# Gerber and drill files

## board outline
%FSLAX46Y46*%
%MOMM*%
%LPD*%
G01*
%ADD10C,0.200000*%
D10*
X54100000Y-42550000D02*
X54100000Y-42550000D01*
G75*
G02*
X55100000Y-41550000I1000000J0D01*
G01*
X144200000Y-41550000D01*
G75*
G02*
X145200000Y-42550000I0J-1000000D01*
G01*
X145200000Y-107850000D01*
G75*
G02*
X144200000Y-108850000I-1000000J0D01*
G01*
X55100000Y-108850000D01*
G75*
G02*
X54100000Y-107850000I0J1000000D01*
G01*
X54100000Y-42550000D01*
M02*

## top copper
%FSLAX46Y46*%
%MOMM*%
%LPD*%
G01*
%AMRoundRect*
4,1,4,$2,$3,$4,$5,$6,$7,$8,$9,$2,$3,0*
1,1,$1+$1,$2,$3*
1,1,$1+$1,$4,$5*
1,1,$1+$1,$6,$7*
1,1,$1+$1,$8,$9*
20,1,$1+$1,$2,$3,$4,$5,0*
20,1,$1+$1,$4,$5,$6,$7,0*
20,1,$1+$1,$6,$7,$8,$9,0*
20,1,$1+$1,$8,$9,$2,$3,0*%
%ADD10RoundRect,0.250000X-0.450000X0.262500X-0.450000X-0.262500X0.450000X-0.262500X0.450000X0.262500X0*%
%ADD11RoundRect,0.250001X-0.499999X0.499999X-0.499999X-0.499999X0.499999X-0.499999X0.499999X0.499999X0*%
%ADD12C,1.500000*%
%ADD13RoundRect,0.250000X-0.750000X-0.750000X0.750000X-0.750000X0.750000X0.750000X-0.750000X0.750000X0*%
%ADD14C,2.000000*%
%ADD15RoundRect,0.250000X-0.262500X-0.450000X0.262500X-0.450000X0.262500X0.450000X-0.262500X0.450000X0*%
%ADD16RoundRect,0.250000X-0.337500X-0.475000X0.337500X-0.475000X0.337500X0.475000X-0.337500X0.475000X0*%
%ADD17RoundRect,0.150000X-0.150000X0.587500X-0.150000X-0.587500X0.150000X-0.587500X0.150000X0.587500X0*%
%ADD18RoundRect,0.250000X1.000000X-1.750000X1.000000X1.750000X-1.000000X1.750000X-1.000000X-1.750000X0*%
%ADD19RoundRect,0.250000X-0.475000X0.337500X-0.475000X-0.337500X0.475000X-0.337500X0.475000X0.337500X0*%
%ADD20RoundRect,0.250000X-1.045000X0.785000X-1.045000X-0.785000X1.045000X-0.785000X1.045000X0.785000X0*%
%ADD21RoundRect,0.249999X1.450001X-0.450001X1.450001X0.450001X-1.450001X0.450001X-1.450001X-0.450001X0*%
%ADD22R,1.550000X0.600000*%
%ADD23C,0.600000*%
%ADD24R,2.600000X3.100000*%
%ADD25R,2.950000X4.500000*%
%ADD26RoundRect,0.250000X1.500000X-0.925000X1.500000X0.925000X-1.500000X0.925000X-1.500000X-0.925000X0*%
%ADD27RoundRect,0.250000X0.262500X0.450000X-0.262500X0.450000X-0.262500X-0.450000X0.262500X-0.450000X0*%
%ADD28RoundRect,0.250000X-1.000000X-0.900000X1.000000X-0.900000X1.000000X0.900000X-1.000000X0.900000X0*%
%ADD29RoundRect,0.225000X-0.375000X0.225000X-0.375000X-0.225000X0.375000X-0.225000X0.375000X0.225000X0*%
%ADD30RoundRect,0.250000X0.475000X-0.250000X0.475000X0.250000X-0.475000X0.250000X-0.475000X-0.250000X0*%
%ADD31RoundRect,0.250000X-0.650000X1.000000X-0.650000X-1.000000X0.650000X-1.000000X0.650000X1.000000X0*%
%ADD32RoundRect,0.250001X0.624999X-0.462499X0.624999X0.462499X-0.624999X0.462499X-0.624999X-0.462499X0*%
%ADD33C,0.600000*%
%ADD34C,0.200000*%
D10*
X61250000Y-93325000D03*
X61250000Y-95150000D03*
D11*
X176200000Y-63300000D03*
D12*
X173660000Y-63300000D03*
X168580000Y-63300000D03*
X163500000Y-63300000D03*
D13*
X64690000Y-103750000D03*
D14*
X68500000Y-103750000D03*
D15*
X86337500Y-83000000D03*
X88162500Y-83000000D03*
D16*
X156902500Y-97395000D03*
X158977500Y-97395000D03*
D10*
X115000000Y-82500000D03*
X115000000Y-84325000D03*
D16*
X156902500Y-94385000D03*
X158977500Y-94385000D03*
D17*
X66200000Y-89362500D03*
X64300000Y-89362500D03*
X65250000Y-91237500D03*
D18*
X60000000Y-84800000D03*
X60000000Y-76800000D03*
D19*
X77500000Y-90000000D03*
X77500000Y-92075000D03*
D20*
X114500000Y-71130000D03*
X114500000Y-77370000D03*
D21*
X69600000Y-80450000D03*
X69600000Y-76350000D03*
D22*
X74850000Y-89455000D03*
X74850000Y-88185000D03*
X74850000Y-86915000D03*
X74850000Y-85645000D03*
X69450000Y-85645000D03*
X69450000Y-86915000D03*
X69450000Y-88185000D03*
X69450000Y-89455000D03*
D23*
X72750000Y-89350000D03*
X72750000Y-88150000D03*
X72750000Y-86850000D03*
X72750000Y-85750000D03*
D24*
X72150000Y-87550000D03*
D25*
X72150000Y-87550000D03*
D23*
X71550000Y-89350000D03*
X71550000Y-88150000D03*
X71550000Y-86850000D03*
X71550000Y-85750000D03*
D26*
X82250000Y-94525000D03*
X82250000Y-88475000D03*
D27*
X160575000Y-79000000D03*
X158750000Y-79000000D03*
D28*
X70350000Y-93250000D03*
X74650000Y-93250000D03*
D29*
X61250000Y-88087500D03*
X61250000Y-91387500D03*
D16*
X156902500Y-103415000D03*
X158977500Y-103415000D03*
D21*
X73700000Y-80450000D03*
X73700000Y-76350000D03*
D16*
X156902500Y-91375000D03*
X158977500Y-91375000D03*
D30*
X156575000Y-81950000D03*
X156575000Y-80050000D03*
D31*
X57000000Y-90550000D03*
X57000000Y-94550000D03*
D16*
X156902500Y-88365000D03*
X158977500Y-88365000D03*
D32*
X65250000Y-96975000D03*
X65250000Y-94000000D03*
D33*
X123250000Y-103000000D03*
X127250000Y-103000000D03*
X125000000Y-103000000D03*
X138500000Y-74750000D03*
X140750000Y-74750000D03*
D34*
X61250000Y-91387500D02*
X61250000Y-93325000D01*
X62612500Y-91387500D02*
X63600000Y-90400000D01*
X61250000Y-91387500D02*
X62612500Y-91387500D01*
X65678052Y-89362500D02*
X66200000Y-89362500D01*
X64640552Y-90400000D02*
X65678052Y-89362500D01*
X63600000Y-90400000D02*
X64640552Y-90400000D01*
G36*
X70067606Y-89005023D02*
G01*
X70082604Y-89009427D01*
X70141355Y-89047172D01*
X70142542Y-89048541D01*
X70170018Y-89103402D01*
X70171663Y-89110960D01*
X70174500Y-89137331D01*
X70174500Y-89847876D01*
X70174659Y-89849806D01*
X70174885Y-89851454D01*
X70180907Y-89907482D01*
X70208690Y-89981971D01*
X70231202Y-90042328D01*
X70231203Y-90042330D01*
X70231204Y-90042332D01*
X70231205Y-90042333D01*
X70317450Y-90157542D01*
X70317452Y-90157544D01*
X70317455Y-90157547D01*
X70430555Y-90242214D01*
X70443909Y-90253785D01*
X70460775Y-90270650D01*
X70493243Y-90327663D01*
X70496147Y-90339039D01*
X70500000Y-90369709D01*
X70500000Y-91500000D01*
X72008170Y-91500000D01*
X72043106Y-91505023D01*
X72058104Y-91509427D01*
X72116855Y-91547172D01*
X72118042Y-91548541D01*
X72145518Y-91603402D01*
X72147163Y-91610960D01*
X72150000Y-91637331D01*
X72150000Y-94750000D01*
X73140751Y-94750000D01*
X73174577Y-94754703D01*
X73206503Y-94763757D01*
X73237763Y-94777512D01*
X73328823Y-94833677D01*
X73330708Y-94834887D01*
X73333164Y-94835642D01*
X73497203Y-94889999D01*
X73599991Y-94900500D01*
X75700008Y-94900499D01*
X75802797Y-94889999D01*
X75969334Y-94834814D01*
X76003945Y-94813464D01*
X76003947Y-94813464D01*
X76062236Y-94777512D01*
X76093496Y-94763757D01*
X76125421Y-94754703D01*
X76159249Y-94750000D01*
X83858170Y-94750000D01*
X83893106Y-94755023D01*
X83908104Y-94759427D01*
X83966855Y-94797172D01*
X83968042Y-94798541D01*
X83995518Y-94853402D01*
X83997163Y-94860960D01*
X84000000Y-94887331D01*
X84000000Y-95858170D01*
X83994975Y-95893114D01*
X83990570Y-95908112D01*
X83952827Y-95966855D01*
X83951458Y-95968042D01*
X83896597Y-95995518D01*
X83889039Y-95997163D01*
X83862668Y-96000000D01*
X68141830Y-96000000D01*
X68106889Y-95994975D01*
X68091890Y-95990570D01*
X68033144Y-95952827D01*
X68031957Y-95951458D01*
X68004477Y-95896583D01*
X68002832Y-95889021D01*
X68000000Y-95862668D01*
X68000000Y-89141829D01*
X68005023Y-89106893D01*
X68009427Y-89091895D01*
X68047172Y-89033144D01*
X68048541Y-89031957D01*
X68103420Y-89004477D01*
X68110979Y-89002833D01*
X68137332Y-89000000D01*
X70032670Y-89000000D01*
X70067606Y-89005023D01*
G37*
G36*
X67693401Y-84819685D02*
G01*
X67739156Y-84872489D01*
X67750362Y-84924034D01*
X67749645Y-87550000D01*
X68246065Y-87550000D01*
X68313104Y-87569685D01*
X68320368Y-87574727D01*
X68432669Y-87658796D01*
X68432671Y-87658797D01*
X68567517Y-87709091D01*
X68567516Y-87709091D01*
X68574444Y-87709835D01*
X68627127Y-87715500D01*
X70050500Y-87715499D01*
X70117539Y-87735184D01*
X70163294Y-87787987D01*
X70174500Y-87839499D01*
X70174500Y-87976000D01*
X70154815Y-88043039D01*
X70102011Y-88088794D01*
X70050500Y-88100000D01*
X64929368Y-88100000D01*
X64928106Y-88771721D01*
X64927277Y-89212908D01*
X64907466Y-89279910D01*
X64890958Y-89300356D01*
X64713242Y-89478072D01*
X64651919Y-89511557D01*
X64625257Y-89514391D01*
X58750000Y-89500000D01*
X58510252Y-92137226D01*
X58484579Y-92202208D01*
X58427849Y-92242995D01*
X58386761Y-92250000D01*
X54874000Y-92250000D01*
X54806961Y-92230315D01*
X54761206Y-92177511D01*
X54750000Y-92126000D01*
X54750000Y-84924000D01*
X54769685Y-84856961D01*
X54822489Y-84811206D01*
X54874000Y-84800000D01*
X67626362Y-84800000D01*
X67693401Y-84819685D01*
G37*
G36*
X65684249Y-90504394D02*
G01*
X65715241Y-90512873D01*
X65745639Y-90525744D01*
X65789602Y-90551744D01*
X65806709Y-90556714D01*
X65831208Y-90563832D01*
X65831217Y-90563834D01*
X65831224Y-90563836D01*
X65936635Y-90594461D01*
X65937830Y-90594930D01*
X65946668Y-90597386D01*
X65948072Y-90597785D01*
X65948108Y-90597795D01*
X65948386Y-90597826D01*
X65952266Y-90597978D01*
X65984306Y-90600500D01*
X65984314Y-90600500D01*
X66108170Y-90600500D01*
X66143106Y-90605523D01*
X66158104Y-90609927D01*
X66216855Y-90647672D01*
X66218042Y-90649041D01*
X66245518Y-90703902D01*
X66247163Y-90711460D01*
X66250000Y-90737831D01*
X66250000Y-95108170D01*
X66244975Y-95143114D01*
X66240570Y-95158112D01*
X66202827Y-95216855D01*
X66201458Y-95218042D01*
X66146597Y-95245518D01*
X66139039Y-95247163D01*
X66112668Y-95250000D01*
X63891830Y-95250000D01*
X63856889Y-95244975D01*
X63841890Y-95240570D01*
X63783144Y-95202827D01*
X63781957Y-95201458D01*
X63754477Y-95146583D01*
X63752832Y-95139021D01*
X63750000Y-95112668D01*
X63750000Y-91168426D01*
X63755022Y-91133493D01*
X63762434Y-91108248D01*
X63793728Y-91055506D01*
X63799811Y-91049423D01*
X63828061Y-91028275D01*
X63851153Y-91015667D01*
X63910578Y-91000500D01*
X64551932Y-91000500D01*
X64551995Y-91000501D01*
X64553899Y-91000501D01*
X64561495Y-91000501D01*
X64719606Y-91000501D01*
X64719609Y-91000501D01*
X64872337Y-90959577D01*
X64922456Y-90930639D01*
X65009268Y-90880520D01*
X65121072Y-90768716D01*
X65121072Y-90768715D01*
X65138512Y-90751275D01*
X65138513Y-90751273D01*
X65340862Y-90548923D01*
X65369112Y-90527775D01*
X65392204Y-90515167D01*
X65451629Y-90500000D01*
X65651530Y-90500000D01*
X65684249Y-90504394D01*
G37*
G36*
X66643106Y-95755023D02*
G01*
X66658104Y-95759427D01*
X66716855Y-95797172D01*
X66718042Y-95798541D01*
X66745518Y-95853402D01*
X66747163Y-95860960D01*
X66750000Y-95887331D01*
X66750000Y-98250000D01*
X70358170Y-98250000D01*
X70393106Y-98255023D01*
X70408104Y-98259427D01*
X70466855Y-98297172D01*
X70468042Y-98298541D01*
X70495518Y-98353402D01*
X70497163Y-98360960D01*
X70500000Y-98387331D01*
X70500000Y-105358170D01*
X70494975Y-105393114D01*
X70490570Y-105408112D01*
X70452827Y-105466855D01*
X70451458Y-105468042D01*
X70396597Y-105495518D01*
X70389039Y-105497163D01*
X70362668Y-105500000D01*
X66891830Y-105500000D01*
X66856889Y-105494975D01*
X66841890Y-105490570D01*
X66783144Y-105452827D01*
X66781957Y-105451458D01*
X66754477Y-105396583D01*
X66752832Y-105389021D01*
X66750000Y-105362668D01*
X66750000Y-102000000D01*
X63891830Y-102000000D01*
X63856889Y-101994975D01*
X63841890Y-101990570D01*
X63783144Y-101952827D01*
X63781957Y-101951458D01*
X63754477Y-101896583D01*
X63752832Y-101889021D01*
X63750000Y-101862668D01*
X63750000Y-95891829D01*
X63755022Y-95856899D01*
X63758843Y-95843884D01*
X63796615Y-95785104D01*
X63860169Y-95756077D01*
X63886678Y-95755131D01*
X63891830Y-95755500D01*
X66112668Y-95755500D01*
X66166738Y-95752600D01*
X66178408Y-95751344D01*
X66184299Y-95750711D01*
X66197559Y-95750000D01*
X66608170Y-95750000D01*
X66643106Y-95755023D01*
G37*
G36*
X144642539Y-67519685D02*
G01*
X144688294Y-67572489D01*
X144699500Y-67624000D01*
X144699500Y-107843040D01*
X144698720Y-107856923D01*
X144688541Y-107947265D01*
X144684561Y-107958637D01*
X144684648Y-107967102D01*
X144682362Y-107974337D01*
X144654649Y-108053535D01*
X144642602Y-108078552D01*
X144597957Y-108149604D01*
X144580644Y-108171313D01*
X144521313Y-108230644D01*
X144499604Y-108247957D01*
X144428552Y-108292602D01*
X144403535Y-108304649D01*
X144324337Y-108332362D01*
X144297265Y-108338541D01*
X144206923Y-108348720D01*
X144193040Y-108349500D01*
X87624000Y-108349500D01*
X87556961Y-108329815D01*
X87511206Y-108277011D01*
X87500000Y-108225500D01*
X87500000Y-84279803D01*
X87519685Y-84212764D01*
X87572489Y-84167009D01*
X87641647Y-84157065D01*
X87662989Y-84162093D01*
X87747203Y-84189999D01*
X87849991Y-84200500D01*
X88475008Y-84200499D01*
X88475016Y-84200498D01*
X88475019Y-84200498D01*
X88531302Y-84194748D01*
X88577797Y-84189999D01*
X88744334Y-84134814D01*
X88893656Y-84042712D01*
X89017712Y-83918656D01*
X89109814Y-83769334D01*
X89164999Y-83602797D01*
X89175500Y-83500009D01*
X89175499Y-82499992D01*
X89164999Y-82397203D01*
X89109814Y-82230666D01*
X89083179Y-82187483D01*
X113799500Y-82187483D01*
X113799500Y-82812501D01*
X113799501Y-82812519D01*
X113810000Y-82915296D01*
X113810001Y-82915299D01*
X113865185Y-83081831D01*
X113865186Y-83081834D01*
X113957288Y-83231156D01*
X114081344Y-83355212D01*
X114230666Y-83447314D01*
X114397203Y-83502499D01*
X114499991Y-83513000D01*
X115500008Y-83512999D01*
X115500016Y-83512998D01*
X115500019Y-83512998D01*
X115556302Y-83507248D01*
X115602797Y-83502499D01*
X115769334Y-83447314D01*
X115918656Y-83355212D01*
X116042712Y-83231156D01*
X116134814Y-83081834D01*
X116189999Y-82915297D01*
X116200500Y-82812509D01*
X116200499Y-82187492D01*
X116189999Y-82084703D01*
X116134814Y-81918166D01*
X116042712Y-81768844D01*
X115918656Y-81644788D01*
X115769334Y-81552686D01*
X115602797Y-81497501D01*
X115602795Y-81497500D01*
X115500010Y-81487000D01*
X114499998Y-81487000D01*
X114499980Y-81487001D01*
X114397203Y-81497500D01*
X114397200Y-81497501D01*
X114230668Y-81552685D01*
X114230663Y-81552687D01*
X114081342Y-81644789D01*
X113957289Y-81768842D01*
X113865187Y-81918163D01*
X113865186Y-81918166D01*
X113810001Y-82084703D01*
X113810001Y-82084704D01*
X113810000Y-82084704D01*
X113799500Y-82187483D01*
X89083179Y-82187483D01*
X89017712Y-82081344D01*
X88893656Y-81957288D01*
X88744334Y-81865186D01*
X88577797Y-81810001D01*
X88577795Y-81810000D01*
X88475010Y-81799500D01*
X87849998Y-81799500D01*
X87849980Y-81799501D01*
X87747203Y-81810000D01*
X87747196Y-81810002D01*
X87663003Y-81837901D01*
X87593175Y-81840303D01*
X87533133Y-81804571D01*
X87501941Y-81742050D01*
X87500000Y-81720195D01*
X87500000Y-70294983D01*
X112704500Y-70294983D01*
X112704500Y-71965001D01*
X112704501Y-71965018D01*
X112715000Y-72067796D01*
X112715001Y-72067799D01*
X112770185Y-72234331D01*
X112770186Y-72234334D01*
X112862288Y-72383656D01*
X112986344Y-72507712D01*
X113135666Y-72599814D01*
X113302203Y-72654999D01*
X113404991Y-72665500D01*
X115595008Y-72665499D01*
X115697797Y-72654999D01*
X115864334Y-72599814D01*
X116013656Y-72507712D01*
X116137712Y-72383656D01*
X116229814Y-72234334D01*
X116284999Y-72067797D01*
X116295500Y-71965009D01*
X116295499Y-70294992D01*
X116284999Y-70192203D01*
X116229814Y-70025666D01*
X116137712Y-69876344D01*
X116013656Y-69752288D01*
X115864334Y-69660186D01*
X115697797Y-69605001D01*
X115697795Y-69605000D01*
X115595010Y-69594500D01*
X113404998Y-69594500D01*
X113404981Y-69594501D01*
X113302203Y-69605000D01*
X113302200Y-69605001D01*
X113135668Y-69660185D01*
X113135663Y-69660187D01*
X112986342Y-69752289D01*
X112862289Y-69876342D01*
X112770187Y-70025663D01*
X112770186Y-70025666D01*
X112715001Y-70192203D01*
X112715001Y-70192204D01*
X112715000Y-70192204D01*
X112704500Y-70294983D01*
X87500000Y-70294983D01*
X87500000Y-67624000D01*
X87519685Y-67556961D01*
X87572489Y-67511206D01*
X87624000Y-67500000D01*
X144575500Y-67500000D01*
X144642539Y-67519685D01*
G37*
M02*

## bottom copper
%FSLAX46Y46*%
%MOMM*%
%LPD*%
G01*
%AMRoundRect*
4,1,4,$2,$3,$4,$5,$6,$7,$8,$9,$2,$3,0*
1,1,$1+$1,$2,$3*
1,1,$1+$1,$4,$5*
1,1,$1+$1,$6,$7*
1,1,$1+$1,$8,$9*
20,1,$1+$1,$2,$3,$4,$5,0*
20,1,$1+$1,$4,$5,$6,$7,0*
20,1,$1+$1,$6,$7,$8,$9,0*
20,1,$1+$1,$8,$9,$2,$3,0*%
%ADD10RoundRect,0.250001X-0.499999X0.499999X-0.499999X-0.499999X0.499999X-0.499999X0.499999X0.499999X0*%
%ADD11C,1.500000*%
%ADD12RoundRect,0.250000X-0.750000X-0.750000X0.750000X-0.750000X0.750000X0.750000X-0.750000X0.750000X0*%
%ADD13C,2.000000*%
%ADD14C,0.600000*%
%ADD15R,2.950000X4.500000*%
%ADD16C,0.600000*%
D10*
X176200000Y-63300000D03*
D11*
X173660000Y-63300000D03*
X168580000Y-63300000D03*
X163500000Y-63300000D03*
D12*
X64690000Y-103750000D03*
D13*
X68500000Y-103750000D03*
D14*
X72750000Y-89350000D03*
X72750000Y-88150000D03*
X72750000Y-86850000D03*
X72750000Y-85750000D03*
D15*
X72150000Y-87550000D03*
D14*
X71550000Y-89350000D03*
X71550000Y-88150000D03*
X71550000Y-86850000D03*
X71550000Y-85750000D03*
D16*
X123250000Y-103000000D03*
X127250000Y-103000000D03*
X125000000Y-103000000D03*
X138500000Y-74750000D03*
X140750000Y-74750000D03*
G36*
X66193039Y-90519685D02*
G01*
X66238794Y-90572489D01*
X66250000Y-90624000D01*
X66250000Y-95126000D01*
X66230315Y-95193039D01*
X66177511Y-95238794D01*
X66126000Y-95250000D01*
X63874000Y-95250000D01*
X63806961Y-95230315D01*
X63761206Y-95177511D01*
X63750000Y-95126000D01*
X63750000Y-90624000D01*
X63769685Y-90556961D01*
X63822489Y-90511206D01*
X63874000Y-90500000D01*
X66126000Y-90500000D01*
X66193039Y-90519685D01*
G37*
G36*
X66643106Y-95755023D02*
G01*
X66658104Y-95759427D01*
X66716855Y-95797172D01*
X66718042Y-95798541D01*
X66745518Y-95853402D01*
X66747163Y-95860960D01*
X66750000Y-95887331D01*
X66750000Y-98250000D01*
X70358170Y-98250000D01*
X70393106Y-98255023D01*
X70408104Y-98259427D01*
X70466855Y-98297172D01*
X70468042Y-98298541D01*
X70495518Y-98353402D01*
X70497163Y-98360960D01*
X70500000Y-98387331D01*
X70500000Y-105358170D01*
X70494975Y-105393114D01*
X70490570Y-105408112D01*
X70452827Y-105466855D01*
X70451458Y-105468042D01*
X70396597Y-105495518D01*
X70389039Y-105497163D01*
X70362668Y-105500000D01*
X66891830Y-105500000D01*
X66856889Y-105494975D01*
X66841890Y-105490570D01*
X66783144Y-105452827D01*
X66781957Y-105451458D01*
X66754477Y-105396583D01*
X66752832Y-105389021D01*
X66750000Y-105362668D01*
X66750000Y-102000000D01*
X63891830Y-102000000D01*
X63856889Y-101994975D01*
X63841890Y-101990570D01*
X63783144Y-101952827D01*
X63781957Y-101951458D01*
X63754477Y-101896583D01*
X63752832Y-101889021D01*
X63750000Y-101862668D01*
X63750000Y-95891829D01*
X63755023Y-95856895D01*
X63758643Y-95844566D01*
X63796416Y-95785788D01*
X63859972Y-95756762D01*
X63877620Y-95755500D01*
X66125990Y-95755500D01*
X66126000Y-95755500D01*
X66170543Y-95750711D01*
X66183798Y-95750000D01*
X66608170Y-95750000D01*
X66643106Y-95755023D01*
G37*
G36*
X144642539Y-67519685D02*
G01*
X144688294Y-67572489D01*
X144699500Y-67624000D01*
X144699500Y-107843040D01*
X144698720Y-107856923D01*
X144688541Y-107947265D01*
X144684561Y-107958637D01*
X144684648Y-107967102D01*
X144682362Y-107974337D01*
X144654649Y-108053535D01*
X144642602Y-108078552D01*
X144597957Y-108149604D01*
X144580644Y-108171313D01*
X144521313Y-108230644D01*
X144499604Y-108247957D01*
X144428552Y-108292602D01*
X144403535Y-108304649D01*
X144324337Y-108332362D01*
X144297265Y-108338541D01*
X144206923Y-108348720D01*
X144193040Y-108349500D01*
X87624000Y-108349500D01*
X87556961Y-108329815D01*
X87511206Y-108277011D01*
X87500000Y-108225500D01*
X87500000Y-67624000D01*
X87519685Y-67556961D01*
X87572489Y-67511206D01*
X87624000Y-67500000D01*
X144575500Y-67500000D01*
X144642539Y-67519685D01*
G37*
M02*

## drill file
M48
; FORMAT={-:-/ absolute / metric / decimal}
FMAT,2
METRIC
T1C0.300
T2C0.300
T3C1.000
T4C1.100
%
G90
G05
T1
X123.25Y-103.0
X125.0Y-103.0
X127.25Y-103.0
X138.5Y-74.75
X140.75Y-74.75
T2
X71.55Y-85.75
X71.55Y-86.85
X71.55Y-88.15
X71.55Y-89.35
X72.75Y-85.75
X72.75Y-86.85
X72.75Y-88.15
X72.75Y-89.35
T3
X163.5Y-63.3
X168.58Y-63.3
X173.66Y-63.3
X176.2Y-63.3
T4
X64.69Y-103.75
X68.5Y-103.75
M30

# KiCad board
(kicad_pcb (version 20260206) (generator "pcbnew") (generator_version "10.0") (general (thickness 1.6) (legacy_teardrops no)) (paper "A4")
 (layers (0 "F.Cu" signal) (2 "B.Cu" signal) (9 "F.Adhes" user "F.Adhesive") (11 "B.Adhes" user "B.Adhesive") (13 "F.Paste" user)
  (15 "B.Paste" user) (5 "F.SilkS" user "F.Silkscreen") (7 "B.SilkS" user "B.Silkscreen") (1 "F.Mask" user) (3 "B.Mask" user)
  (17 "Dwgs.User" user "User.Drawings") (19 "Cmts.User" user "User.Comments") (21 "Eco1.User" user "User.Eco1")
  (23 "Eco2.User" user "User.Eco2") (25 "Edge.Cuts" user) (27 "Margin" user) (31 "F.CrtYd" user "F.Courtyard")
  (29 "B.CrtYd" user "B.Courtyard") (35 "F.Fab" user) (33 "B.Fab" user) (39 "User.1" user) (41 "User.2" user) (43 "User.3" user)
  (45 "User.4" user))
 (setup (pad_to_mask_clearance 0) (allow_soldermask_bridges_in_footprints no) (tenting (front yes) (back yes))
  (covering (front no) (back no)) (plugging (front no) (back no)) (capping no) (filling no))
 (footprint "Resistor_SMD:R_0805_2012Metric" (layer "F.Cu") (at 61.25 94.2375 -90)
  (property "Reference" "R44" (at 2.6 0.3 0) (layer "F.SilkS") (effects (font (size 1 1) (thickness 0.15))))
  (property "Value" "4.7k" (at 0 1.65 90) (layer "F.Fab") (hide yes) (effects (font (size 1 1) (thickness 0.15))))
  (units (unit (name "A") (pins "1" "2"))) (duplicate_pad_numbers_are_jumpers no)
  (pad "1" smd roundrect (at -0.9125 0 270) (size 1.025 1.4) (layers "F.Cu" "F.Mask" "F.Paste") (roundrect_rratio 0.243902)
   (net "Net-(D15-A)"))
  (pad "2" smd roundrect (at 0.9125 0 270) (size 1.025 1.4) (layers "F.Cu" "F.Mask" "F.Paste") (roundrect_rratio 0.243902) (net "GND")))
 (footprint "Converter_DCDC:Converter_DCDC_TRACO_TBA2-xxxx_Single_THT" (layer "F.Cu") (at 176.2 63.3 -90)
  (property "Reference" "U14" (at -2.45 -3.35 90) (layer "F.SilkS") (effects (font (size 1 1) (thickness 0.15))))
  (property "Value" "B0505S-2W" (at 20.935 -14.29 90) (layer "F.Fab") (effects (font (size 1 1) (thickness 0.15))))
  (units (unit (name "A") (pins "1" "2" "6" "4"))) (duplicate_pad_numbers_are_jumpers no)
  (pad "1" thru_hole roundrect (at 0 0 270) (size 1.5 1.5) (drill 1) (layers "*.Cu" "*.Mask") (remove_unused_layers no)
   (roundrect_rratio 0.166667) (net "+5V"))
  (pad "2" thru_hole circle (at 0 2.54 270) (size 1.5 1.5) (drill 1) (layers "*.Cu" "*.Mask") (remove_unused_layers no) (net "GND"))
  (pad "4" thru_hole circle (at 0 7.62 270) (size 1.5 1.5) (drill 1) (layers "*.Cu" "*.Mask") (remove_unused_layers no) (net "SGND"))
  (pad "6" thru_hole circle (at 0 12.7 270) (size 1.5 1.5) (drill 1) (layers "*.Cu" "*.Mask") (remove_unused_layers no) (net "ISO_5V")))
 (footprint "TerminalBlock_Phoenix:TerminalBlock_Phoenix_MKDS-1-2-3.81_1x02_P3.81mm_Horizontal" (layer "F.Cu") (at 64.69 103.75)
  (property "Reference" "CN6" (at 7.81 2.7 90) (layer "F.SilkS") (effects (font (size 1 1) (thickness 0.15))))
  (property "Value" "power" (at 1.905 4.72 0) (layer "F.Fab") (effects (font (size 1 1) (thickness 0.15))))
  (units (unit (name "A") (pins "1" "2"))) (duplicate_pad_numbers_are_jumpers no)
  (pad "1" thru_hole roundrect (at 0 0) (size 2 2) (drill 1.1) (layers "*.Cu" "*.Mask") (remove_unused_layers no) (roundrect_rratio 0.125)
   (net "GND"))
  (pad "2" thru_hole circle (at 3.81 0) (size 2 2) (drill 1.1) (layers "*.Cu" "*.Mask") (remove_unused_layers no) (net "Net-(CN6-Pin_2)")))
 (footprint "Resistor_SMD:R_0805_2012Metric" (layer "F.Cu") (at 87.25 83)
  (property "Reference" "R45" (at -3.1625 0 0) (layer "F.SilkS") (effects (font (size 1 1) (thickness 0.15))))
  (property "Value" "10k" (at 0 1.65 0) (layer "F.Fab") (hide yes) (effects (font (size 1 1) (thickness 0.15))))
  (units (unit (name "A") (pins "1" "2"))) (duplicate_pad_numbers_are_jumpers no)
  (pad "1" smd roundrect (at -0.9125 0) (size 1.025 1.4) (layers "F.Cu" "F.Mask" "F.Paste") (roundrect_rratio 0.243902) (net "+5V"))
  (pad "2" smd roundrect (at 0.9125 0) (size 1.025 1.4) (layers "F.Cu" "F.Mask" "F.Paste") (roundrect_rratio 0.243902)
   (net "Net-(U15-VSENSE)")))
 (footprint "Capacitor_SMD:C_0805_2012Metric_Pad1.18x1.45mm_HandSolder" (layer "F.Cu") (at 157.94 97.395)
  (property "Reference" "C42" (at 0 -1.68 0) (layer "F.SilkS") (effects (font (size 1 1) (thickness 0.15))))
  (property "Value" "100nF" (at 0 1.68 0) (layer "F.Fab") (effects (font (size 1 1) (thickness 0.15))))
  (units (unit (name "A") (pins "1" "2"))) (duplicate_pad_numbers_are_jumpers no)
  (pad "1" smd roundrect (at -1.0375 0) (size 1.175 1.45) (layers "F.Cu" "F.Mask" "F.Paste") (roundrect_rratio 0.212766) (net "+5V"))
  (pad "2" smd roundrect (at 1.0375 0) (size 1.175 1.45) (layers "F.Cu" "F.Mask" "F.Paste") (roundrect_rratio 0.212766) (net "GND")))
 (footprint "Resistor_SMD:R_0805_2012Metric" (layer "F.Cu") (at 115 83.4125 -90)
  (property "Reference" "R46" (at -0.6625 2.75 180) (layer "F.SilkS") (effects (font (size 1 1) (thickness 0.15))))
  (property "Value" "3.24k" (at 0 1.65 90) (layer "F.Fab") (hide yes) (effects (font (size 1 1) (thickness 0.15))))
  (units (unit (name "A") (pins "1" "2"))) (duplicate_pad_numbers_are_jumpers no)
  (pad "1" smd roundrect (at -0.9125 0 270) (size 1.025 1.4) (layers "F.Cu" "F.Mask" "F.Paste") (roundrect_rratio 0.243902)
   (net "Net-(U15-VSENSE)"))
  (pad "2" smd roundrect (at 0.9125 0 270) (size 1.025 1.4) (layers "F.Cu" "F.Mask" "F.Paste") (roundrect_rratio 0.243902) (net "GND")))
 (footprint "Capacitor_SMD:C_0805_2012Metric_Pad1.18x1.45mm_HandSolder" (layer "F.Cu") (at 157.94 94.385)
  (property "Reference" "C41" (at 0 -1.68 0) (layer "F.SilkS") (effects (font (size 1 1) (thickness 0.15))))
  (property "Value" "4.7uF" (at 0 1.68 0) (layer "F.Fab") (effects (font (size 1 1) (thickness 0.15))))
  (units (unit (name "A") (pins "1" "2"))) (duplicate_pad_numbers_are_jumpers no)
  (pad "1" smd roundrect (at -1.0375 0) (size 1.175 1.45) (layers "F.Cu" "F.Mask" "F.Paste") (roundrect_rratio 0.212766) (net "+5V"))
  (pad "2" smd roundrect (at 1.0375 0) (size 1.175 1.45) (layers "F.Cu" "F.Mask" "F.Paste") (roundrect_rratio 0.212766) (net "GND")))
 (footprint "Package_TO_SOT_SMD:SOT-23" (layer "F.Cu") (at 65.25 90.3 -90)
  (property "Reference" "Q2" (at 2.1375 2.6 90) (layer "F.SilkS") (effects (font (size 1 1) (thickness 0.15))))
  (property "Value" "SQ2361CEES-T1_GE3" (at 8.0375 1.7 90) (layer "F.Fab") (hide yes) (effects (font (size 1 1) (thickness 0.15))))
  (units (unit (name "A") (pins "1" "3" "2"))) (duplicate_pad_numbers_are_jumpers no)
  (pad "1" smd roundrect (at -0.9375 -0.95 270) (size 1.475 0.6) (layers "F.Cu" "F.Mask" "F.Paste") (roundrect_rratio 0.25)
   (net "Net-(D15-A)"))
  (pad "2" smd roundrect (at -0.9375 0.95 270) (size 1.475 0.6) (layers "F.Cu" "F.Mask" "F.Paste") (roundrect_rratio 0.25)
   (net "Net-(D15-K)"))
  (pad "3" smd roundrect (at 0.9375 0 270) (size 1.475 0.6) (layers "F.Cu" "F.Mask" "F.Paste") (roundrect_rratio 0.25) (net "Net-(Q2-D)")))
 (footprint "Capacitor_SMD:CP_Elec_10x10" (layer "F.Cu") (at 60 80.8 90)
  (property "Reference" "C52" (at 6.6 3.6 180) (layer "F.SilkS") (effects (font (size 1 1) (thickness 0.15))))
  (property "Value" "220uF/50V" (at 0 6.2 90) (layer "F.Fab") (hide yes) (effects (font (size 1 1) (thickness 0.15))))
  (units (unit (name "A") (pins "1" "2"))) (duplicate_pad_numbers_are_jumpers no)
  (pad "1" smd roundrect (at -4 0 90) (size 4 2.5) (layers "F.Cu" "F.Mask" "F.Paste") (roundrect_rratio 0.1) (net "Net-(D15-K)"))
  (pad "2" smd roundrect (at 4 0 90) (size 4 2.5) (layers "F.Cu" "F.Mask" "F.Paste") (roundrect_rratio 0.1) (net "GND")))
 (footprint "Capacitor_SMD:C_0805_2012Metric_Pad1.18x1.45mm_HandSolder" (layer "F.Cu") (at 77.5 91.0375 -90)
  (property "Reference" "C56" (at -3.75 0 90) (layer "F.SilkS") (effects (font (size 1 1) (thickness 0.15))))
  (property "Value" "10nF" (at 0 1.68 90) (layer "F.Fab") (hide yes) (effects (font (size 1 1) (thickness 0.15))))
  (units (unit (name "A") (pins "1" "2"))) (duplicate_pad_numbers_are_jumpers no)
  (pad "1" smd roundrect (at -1.0375 0 270) (size 1.175 1.45) (layers "F.Cu" "F.Mask" "F.Paste") (roundrect_rratio 0.212766)
   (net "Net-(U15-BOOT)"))
  (pad "2" smd roundrect (at 1.0375 0 270) (size 1.175 1.45) (layers "F.Cu" "F.Mask" "F.Paste") (roundrect_rratio 0.212766)
   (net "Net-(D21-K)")))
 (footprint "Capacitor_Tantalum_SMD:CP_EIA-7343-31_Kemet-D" (layer "F.Cu") (at 114.5 74.25 -90)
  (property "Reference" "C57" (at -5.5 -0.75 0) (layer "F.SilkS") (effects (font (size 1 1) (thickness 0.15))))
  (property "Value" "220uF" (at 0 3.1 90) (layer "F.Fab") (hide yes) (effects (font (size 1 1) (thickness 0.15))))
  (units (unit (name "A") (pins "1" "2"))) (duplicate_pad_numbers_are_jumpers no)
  (pad "1" smd roundrect (at -3.12 0 270) (size 2.07 2.59) (layers "F.Cu" "F.Mask" "F.Paste") (roundrect_rratio 0.120773) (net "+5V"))
  (pad "2" smd roundrect (at 3.12 0 270) (size 2.07 2.59) (layers "F.Cu" "F.Mask" "F.Paste") (roundrect_rratio 0.120773) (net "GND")))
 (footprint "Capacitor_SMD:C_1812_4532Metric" (layer "F.Cu") (at 69.6 78.4 90)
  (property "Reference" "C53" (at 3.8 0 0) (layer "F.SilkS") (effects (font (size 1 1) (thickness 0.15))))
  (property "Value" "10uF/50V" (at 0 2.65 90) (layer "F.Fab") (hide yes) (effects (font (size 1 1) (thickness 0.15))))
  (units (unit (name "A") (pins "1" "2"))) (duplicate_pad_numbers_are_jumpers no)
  (pad "1" smd roundrect (at -2.05 0 90) (size 1.4 3.4) (layers "F.Cu" "F.Mask" "F.Paste") (roundrect_rratio 0.178571) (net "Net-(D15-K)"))
  (pad "2" smd roundrect (at 2.05 0 90) (size 1.4 3.4) (layers "F.Cu" "F.Mask" "F.Paste") (roundrect_rratio 0.178571) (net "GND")))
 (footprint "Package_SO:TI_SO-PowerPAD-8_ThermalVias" (layer "F.Cu") (at 72.15 87.55 180)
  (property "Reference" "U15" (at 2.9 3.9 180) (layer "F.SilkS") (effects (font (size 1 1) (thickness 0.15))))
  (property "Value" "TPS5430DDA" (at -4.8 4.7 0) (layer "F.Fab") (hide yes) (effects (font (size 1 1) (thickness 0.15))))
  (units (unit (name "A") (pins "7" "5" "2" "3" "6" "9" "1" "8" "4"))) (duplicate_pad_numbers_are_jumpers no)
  (pad "1" smd rect (at -2.7 -1.905 180) (size 1.55 0.6) (layers "F.Cu" "F.Mask" "F.Paste") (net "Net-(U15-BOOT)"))
  (pad "2" smd rect (at -2.7 -0.635 180) (size 1.55 0.6) (layers "F.Cu" "F.Mask" "F.Paste") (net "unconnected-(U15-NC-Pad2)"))
  (pad "3" smd rect (at -2.7 0.635 180) (size 1.55 0.6) (layers "F.Cu" "F.Mask" "F.Paste") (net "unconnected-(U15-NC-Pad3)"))
  (pad "4" smd rect (at -2.7 1.905 180) (size 1.55 0.6) (layers "F.Cu" "F.Mask" "F.Paste") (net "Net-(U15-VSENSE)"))
  (pad "5" smd rect (at 2.7 1.905 180) (size 1.55 0.6) (layers "F.Cu" "F.Mask" "F.Paste") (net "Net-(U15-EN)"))
  (pad "6" smd rect (at 2.7 0.635 180) (size 1.55 0.6) (layers "F.Cu" "F.Mask" "F.Paste") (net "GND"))
  (pad "7" smd rect (at 2.7 -0.635 180) (size 1.55 0.6) (layers "F.Cu" "F.Mask" "F.Paste") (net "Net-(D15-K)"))
  (pad "8" smd rect (at 2.7 -1.905 180) (size 1.55 0.6) (layers "F.Cu" "F.Mask" "F.Paste") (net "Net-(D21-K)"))
  (pad "9" thru_hole circle (at -0.6 -1.8 180) (size 0.6 0.6) (drill 0.3) (layers "*.Cu") (remove_unused_layers no) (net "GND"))
  (pad "9" thru_hole circle (at -0.6 -0.6 180) (size 0.6 0.6) (drill 0.3) (layers "*.Cu") (remove_unused_layers no) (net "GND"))
  (pad "9" thru_hole circle (at -0.6 0.7 180) (size 0.6 0.6) (drill 0.3) (layers "*.Cu") (remove_unused_layers no) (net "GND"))
  (pad "9" thru_hole circle (at -0.6 1.8 180) (size 0.6 0.6) (drill 0.3) (layers "*.Cu") (remove_unused_layers no) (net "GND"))
  (pad "9" smd rect (at 0 0 180) (size 2.6 3.1) (layers "F.Cu" "F.Mask" "F.Paste") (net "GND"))
  (pad "9" smd rect (at 0 0 180) (size 2.95 4.5) (layers "F.Cu") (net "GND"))
  (pad "9" smd rect (at 0 0 180) (size 2.95 4.5) (layers "B.Cu") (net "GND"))
  (pad "9" thru_hole circle (at 0.6 -1.8 180) (size 0.6 0.6) (drill 0.3) (layers "*.Cu") (remove_unused_layers no) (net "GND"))
  (pad "9" thru_hole circle (at 0.6 -0.6 180) (size 0.6 0.6) (drill 0.3) (layers "*.Cu") (remove_unused_layers no) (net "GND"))
  (pad "9" thru_hole circle (at 0.6 0.7 180) (size 0.6 0.6) (drill 0.3) (layers "*.Cu") (remove_unused_layers no) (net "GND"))
  (pad "9" thru_hole circle (at 0.6 1.8 180) (size 0.6 0.6) (drill 0.3) (layers "*.Cu") (remove_unused_layers no) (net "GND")))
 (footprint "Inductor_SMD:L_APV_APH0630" (layer "F.Cu") (at 82.25 91.5 90)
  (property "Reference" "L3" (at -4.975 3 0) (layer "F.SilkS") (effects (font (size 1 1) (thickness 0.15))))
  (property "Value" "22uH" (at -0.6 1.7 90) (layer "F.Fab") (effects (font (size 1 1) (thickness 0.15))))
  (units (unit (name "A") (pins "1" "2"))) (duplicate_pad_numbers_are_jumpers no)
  (pad "1" smd roundrect (at -3.025 0 90) (size 2.35 3.5) (layers "F.Cu" "F.Mask" "F.Paste") (roundrect_rratio 0.106383) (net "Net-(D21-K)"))
  (pad "2" smd roundrect (at 3.025 0 90) (size 2.35 3.5) (layers "F.Cu" "F.Mask" "F.Paste") (roundrect_rratio 0.106383) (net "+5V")))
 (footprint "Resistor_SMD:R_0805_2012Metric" (layer "F.Cu") (at 159.6625 79 180)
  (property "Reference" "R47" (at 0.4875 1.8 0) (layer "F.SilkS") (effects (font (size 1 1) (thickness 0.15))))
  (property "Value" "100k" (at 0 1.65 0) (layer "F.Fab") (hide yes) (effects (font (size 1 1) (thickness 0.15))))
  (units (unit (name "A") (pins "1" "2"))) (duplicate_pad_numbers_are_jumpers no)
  (pad "1" smd roundrect (at -0.9125 0 180) (size 1.025 1.4) (layers "F.Cu" "F.Mask" "F.Paste") (roundrect_rratio 0.243902)
   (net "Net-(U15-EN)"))
  (pad "2" smd roundrect (at 0.9125 0 180) (size 1.025 1.4) (layers "F.Cu" "F.Mask" "F.Paste") (roundrect_rratio 0.243902)
   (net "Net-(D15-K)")))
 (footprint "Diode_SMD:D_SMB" (layer "F.Cu") (at 72.5 93.25)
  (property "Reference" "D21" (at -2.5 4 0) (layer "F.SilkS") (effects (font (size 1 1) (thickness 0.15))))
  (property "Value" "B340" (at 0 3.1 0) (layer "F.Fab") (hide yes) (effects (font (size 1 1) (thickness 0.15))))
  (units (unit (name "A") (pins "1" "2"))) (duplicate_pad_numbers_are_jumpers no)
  (pad "1" smd roundrect (at -2.15 0) (size 2.5 2.3) (layers "F.Cu" "F.Mask" "F.Paste") (roundrect_rratio 0.1086956522) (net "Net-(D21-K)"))
  (pad "2" smd roundrect (at 2.15 0) (size 2.5 2.3) (layers "F.Cu" "F.Mask" "F.Paste") (roundrect_rratio 0.1086956522) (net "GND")))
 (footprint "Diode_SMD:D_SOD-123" (layer "F.Cu") (at 61.25 89.7375 -90)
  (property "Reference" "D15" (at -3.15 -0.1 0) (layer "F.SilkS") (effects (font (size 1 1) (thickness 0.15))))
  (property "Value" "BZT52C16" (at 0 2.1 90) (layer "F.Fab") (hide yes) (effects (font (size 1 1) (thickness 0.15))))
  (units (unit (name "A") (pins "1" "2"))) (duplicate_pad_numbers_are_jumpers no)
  (pad "1" smd roundrect (at -1.65 0 270) (size 0.9 1.2) (layers "F.Cu" "F.Mask" "F.Paste") (roundrect_rratio 0.25) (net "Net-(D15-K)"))
  (pad "2" smd roundrect (at 1.65 0 270) (size 0.9 1.2) (layers "F.Cu" "F.Mask" "F.Paste") (roundrect_rratio 0.25) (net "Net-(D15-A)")))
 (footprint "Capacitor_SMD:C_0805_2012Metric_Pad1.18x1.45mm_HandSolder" (layer "F.Cu") (at 157.94 103.415)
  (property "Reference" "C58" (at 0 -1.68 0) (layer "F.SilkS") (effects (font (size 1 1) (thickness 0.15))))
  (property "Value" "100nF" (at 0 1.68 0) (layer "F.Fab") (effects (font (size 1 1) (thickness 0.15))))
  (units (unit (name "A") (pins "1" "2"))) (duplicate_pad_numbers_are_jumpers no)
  (pad "1" smd roundrect (at -1.0375 0) (size 1.175 1.45) (layers "F.Cu" "F.Mask" "F.Paste") (roundrect_rratio 0.212766) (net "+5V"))
  (pad "2" smd roundrect (at 1.0375 0) (size 1.175 1.45) (layers "F.Cu" "F.Mask" "F.Paste") (roundrect_rratio 0.212766) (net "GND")))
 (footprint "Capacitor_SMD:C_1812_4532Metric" (layer "F.Cu") (at 73.7 78.4 90)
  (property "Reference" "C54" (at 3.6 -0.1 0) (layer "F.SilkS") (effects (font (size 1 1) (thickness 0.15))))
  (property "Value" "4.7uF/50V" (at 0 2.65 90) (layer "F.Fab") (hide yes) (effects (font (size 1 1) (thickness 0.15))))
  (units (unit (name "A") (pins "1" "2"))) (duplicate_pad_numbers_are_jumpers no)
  (pad "1" smd roundrect (at -2.05 0 90) (size 1.4 3.4) (layers "F.Cu" "F.Mask" "F.Paste") (roundrect_rratio 0.178571) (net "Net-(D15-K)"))
  (pad "2" smd roundrect (at 2.05 0 90) (size 1.4 3.4) (layers "F.Cu" "F.Mask" "F.Paste") (roundrect_rratio 0.178571) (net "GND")))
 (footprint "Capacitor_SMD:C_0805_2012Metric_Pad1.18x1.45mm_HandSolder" (layer "F.Cu") (at 157.94 91.375)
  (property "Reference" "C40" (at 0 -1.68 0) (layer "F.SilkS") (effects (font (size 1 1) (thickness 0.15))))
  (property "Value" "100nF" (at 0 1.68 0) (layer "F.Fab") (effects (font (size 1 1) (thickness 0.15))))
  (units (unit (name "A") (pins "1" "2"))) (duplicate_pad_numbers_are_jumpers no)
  (pad "1" smd roundrect (at -1.0375 0) (size 1.175 1.45) (layers "F.Cu" "F.Mask" "F.Paste") (roundrect_rratio 0.212766) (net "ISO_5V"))
  (pad "2" smd roundrect (at 1.0375 0) (size 1.175 1.45) (layers "F.Cu" "F.Mask" "F.Paste") (roundrect_rratio 0.212766) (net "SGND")))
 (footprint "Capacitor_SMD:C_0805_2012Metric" (layer "F.Cu") (at 156.575 81 90)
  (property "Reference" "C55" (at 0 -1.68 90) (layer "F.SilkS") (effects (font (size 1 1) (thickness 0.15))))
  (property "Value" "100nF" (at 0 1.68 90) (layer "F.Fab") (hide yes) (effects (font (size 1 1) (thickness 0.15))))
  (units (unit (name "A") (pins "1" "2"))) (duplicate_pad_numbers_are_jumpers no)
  (pad "1" smd roundrect (at -0.95 0 90) (size 1 1.45) (layers "F.Cu" "F.Mask" "F.Paste") (roundrect_rratio 0.25) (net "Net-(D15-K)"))
  (pad "2" smd roundrect (at 0.95 0 90) (size 1 1.45) (layers "F.Cu" "F.Mask" "F.Paste") (roundrect_rratio 0.25) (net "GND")))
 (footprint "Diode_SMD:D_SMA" (layer "F.Cu") (at 57 92.55 -90)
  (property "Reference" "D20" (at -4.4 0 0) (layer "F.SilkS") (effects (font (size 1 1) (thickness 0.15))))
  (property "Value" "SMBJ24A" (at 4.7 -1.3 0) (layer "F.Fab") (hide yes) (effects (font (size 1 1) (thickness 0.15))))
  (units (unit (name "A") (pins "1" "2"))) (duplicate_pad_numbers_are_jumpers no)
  (pad "1" smd roundrect (at -2 0 270) (size 2.5 1.8) (layers "F.Cu" "F.Mask" "F.Paste") (roundrect_rratio 0.1388888889) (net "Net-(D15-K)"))
  (pad "2" smd roundrect (at 2 0 270) (size 2.5 1.8) (layers "F.Cu" "F.Mask" "F.Paste") (roundrect_rratio 0.1388888889) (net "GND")))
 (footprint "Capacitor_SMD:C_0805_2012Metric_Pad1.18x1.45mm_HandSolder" (layer "F.Cu") (at 157.94 88.365)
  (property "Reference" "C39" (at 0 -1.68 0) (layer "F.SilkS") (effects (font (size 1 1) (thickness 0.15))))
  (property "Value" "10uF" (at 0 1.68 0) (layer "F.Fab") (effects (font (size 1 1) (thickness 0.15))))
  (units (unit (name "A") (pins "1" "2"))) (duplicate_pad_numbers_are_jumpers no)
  (pad "1" smd roundrect (at -1.0375 0) (size 1.175 1.45) (layers "F.Cu" "F.Mask" "F.Paste") (roundrect_rratio 0.212766) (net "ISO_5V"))
  (pad "2" smd roundrect (at 1.0375 0) (size 1.175 1.45) (layers "F.Cu" "F.Mask" "F.Paste") (roundrect_rratio 0.212766) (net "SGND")))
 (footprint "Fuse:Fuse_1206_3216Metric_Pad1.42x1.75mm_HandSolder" (layer "F.Cu") (at 65.25 95.4875 90)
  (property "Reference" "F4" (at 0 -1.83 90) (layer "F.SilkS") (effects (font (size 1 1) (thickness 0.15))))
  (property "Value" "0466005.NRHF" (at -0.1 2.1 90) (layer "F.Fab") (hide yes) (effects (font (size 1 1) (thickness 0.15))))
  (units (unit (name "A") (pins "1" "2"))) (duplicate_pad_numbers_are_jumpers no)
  (pad "1" smd roundrect (at -1.4875 0 90) (size 1.425 1.75) (layers "F.Cu" "F.Mask" "F.Paste") (roundrect_rratio 0.175439)
   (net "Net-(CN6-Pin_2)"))
  (pad "2" smd roundrect (at 1.4875 0 90) (size 1.425 1.75) (layers "F.Cu" "F.Mask" "F.Paste") (roundrect_rratio 0.175439)
   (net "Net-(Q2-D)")))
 (gr_rect (start 54.1 41.55) (end 145.2 108.85) (radius 1) (stroke (width 0.2) (type solid)) (fill no) (layer "Edge.Cuts"))
 (via (at 123.25 103) (size 0.6) (drill 0.3) (layers "F.Cu" "B.Cu") (free yes) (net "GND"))
 (via (at 127.25 103) (size 0.6) (drill 0.3) (layers "F.Cu" "B.Cu") (free yes) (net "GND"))
 (via (at 125 103) (size 0.6) (drill 0.3) (layers "F.Cu" "B.Cu") (free yes) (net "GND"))
 (via (at 138.5 74.75) (size 0.6) (drill 0.3) (layers "F.Cu" "B.Cu") (free yes) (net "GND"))
 (via (at 140.75 74.75) (size 0.6) (drill 0.3) (layers "F.Cu" "B.Cu") (free yes) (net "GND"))
 (segment (start 61.25 91.3875) (end 61.25 93.325) (width 0.2) (layer "F.Cu") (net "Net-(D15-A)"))
 (segment (start 62.6125 91.3875) (end 63.6 90.4) (width 0.2) (layer "F.Cu") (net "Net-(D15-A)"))
 (segment (start 61.25 91.3875) (end 62.6125 91.3875) (width 0.2) (layer "F.Cu") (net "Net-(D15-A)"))
 (segment (start 65.678052 89.3625) (end 66.2 89.3625) (width 0.2) (layer "F.Cu") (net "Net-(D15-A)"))
 (segment (start 64.640552 90.4) (end 65.678052 89.3625) (width 0.2) (layer "F.Cu") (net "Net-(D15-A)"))
 (segment (start 63.6 90.4) (end 64.640552 90.4) (width 0.2) (layer "F.Cu") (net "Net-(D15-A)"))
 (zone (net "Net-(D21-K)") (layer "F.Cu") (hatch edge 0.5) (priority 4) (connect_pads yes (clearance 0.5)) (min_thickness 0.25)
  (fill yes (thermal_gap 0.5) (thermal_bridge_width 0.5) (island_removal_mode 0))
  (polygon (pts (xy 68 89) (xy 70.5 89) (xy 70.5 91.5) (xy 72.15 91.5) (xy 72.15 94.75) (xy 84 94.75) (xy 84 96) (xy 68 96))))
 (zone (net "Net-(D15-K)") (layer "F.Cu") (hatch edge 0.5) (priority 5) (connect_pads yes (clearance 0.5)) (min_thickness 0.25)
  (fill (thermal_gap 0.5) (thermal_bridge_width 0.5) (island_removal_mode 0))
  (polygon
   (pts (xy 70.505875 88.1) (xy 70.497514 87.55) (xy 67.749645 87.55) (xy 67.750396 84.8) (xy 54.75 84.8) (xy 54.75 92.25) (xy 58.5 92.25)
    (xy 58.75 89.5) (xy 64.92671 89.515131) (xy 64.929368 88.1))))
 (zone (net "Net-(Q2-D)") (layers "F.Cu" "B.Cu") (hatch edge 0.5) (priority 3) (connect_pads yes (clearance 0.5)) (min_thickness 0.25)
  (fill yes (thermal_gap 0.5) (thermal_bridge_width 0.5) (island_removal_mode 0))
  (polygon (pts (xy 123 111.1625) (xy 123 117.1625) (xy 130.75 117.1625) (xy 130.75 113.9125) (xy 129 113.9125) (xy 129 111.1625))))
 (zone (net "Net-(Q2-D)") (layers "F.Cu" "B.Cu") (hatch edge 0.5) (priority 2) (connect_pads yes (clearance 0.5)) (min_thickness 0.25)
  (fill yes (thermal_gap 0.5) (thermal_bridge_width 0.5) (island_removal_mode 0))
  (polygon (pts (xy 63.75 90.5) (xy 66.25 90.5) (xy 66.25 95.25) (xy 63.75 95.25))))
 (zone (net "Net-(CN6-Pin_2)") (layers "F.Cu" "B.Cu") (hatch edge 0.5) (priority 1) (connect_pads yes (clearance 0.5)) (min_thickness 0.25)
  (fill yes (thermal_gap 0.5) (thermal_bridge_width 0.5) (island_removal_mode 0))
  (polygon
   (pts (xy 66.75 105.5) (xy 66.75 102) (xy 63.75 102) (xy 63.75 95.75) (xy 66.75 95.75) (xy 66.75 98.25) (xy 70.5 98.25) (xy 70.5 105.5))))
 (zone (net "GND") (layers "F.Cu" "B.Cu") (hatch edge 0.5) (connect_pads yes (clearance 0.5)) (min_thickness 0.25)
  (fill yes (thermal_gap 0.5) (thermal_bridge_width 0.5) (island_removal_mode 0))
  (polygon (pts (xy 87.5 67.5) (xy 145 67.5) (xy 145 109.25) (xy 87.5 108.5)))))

